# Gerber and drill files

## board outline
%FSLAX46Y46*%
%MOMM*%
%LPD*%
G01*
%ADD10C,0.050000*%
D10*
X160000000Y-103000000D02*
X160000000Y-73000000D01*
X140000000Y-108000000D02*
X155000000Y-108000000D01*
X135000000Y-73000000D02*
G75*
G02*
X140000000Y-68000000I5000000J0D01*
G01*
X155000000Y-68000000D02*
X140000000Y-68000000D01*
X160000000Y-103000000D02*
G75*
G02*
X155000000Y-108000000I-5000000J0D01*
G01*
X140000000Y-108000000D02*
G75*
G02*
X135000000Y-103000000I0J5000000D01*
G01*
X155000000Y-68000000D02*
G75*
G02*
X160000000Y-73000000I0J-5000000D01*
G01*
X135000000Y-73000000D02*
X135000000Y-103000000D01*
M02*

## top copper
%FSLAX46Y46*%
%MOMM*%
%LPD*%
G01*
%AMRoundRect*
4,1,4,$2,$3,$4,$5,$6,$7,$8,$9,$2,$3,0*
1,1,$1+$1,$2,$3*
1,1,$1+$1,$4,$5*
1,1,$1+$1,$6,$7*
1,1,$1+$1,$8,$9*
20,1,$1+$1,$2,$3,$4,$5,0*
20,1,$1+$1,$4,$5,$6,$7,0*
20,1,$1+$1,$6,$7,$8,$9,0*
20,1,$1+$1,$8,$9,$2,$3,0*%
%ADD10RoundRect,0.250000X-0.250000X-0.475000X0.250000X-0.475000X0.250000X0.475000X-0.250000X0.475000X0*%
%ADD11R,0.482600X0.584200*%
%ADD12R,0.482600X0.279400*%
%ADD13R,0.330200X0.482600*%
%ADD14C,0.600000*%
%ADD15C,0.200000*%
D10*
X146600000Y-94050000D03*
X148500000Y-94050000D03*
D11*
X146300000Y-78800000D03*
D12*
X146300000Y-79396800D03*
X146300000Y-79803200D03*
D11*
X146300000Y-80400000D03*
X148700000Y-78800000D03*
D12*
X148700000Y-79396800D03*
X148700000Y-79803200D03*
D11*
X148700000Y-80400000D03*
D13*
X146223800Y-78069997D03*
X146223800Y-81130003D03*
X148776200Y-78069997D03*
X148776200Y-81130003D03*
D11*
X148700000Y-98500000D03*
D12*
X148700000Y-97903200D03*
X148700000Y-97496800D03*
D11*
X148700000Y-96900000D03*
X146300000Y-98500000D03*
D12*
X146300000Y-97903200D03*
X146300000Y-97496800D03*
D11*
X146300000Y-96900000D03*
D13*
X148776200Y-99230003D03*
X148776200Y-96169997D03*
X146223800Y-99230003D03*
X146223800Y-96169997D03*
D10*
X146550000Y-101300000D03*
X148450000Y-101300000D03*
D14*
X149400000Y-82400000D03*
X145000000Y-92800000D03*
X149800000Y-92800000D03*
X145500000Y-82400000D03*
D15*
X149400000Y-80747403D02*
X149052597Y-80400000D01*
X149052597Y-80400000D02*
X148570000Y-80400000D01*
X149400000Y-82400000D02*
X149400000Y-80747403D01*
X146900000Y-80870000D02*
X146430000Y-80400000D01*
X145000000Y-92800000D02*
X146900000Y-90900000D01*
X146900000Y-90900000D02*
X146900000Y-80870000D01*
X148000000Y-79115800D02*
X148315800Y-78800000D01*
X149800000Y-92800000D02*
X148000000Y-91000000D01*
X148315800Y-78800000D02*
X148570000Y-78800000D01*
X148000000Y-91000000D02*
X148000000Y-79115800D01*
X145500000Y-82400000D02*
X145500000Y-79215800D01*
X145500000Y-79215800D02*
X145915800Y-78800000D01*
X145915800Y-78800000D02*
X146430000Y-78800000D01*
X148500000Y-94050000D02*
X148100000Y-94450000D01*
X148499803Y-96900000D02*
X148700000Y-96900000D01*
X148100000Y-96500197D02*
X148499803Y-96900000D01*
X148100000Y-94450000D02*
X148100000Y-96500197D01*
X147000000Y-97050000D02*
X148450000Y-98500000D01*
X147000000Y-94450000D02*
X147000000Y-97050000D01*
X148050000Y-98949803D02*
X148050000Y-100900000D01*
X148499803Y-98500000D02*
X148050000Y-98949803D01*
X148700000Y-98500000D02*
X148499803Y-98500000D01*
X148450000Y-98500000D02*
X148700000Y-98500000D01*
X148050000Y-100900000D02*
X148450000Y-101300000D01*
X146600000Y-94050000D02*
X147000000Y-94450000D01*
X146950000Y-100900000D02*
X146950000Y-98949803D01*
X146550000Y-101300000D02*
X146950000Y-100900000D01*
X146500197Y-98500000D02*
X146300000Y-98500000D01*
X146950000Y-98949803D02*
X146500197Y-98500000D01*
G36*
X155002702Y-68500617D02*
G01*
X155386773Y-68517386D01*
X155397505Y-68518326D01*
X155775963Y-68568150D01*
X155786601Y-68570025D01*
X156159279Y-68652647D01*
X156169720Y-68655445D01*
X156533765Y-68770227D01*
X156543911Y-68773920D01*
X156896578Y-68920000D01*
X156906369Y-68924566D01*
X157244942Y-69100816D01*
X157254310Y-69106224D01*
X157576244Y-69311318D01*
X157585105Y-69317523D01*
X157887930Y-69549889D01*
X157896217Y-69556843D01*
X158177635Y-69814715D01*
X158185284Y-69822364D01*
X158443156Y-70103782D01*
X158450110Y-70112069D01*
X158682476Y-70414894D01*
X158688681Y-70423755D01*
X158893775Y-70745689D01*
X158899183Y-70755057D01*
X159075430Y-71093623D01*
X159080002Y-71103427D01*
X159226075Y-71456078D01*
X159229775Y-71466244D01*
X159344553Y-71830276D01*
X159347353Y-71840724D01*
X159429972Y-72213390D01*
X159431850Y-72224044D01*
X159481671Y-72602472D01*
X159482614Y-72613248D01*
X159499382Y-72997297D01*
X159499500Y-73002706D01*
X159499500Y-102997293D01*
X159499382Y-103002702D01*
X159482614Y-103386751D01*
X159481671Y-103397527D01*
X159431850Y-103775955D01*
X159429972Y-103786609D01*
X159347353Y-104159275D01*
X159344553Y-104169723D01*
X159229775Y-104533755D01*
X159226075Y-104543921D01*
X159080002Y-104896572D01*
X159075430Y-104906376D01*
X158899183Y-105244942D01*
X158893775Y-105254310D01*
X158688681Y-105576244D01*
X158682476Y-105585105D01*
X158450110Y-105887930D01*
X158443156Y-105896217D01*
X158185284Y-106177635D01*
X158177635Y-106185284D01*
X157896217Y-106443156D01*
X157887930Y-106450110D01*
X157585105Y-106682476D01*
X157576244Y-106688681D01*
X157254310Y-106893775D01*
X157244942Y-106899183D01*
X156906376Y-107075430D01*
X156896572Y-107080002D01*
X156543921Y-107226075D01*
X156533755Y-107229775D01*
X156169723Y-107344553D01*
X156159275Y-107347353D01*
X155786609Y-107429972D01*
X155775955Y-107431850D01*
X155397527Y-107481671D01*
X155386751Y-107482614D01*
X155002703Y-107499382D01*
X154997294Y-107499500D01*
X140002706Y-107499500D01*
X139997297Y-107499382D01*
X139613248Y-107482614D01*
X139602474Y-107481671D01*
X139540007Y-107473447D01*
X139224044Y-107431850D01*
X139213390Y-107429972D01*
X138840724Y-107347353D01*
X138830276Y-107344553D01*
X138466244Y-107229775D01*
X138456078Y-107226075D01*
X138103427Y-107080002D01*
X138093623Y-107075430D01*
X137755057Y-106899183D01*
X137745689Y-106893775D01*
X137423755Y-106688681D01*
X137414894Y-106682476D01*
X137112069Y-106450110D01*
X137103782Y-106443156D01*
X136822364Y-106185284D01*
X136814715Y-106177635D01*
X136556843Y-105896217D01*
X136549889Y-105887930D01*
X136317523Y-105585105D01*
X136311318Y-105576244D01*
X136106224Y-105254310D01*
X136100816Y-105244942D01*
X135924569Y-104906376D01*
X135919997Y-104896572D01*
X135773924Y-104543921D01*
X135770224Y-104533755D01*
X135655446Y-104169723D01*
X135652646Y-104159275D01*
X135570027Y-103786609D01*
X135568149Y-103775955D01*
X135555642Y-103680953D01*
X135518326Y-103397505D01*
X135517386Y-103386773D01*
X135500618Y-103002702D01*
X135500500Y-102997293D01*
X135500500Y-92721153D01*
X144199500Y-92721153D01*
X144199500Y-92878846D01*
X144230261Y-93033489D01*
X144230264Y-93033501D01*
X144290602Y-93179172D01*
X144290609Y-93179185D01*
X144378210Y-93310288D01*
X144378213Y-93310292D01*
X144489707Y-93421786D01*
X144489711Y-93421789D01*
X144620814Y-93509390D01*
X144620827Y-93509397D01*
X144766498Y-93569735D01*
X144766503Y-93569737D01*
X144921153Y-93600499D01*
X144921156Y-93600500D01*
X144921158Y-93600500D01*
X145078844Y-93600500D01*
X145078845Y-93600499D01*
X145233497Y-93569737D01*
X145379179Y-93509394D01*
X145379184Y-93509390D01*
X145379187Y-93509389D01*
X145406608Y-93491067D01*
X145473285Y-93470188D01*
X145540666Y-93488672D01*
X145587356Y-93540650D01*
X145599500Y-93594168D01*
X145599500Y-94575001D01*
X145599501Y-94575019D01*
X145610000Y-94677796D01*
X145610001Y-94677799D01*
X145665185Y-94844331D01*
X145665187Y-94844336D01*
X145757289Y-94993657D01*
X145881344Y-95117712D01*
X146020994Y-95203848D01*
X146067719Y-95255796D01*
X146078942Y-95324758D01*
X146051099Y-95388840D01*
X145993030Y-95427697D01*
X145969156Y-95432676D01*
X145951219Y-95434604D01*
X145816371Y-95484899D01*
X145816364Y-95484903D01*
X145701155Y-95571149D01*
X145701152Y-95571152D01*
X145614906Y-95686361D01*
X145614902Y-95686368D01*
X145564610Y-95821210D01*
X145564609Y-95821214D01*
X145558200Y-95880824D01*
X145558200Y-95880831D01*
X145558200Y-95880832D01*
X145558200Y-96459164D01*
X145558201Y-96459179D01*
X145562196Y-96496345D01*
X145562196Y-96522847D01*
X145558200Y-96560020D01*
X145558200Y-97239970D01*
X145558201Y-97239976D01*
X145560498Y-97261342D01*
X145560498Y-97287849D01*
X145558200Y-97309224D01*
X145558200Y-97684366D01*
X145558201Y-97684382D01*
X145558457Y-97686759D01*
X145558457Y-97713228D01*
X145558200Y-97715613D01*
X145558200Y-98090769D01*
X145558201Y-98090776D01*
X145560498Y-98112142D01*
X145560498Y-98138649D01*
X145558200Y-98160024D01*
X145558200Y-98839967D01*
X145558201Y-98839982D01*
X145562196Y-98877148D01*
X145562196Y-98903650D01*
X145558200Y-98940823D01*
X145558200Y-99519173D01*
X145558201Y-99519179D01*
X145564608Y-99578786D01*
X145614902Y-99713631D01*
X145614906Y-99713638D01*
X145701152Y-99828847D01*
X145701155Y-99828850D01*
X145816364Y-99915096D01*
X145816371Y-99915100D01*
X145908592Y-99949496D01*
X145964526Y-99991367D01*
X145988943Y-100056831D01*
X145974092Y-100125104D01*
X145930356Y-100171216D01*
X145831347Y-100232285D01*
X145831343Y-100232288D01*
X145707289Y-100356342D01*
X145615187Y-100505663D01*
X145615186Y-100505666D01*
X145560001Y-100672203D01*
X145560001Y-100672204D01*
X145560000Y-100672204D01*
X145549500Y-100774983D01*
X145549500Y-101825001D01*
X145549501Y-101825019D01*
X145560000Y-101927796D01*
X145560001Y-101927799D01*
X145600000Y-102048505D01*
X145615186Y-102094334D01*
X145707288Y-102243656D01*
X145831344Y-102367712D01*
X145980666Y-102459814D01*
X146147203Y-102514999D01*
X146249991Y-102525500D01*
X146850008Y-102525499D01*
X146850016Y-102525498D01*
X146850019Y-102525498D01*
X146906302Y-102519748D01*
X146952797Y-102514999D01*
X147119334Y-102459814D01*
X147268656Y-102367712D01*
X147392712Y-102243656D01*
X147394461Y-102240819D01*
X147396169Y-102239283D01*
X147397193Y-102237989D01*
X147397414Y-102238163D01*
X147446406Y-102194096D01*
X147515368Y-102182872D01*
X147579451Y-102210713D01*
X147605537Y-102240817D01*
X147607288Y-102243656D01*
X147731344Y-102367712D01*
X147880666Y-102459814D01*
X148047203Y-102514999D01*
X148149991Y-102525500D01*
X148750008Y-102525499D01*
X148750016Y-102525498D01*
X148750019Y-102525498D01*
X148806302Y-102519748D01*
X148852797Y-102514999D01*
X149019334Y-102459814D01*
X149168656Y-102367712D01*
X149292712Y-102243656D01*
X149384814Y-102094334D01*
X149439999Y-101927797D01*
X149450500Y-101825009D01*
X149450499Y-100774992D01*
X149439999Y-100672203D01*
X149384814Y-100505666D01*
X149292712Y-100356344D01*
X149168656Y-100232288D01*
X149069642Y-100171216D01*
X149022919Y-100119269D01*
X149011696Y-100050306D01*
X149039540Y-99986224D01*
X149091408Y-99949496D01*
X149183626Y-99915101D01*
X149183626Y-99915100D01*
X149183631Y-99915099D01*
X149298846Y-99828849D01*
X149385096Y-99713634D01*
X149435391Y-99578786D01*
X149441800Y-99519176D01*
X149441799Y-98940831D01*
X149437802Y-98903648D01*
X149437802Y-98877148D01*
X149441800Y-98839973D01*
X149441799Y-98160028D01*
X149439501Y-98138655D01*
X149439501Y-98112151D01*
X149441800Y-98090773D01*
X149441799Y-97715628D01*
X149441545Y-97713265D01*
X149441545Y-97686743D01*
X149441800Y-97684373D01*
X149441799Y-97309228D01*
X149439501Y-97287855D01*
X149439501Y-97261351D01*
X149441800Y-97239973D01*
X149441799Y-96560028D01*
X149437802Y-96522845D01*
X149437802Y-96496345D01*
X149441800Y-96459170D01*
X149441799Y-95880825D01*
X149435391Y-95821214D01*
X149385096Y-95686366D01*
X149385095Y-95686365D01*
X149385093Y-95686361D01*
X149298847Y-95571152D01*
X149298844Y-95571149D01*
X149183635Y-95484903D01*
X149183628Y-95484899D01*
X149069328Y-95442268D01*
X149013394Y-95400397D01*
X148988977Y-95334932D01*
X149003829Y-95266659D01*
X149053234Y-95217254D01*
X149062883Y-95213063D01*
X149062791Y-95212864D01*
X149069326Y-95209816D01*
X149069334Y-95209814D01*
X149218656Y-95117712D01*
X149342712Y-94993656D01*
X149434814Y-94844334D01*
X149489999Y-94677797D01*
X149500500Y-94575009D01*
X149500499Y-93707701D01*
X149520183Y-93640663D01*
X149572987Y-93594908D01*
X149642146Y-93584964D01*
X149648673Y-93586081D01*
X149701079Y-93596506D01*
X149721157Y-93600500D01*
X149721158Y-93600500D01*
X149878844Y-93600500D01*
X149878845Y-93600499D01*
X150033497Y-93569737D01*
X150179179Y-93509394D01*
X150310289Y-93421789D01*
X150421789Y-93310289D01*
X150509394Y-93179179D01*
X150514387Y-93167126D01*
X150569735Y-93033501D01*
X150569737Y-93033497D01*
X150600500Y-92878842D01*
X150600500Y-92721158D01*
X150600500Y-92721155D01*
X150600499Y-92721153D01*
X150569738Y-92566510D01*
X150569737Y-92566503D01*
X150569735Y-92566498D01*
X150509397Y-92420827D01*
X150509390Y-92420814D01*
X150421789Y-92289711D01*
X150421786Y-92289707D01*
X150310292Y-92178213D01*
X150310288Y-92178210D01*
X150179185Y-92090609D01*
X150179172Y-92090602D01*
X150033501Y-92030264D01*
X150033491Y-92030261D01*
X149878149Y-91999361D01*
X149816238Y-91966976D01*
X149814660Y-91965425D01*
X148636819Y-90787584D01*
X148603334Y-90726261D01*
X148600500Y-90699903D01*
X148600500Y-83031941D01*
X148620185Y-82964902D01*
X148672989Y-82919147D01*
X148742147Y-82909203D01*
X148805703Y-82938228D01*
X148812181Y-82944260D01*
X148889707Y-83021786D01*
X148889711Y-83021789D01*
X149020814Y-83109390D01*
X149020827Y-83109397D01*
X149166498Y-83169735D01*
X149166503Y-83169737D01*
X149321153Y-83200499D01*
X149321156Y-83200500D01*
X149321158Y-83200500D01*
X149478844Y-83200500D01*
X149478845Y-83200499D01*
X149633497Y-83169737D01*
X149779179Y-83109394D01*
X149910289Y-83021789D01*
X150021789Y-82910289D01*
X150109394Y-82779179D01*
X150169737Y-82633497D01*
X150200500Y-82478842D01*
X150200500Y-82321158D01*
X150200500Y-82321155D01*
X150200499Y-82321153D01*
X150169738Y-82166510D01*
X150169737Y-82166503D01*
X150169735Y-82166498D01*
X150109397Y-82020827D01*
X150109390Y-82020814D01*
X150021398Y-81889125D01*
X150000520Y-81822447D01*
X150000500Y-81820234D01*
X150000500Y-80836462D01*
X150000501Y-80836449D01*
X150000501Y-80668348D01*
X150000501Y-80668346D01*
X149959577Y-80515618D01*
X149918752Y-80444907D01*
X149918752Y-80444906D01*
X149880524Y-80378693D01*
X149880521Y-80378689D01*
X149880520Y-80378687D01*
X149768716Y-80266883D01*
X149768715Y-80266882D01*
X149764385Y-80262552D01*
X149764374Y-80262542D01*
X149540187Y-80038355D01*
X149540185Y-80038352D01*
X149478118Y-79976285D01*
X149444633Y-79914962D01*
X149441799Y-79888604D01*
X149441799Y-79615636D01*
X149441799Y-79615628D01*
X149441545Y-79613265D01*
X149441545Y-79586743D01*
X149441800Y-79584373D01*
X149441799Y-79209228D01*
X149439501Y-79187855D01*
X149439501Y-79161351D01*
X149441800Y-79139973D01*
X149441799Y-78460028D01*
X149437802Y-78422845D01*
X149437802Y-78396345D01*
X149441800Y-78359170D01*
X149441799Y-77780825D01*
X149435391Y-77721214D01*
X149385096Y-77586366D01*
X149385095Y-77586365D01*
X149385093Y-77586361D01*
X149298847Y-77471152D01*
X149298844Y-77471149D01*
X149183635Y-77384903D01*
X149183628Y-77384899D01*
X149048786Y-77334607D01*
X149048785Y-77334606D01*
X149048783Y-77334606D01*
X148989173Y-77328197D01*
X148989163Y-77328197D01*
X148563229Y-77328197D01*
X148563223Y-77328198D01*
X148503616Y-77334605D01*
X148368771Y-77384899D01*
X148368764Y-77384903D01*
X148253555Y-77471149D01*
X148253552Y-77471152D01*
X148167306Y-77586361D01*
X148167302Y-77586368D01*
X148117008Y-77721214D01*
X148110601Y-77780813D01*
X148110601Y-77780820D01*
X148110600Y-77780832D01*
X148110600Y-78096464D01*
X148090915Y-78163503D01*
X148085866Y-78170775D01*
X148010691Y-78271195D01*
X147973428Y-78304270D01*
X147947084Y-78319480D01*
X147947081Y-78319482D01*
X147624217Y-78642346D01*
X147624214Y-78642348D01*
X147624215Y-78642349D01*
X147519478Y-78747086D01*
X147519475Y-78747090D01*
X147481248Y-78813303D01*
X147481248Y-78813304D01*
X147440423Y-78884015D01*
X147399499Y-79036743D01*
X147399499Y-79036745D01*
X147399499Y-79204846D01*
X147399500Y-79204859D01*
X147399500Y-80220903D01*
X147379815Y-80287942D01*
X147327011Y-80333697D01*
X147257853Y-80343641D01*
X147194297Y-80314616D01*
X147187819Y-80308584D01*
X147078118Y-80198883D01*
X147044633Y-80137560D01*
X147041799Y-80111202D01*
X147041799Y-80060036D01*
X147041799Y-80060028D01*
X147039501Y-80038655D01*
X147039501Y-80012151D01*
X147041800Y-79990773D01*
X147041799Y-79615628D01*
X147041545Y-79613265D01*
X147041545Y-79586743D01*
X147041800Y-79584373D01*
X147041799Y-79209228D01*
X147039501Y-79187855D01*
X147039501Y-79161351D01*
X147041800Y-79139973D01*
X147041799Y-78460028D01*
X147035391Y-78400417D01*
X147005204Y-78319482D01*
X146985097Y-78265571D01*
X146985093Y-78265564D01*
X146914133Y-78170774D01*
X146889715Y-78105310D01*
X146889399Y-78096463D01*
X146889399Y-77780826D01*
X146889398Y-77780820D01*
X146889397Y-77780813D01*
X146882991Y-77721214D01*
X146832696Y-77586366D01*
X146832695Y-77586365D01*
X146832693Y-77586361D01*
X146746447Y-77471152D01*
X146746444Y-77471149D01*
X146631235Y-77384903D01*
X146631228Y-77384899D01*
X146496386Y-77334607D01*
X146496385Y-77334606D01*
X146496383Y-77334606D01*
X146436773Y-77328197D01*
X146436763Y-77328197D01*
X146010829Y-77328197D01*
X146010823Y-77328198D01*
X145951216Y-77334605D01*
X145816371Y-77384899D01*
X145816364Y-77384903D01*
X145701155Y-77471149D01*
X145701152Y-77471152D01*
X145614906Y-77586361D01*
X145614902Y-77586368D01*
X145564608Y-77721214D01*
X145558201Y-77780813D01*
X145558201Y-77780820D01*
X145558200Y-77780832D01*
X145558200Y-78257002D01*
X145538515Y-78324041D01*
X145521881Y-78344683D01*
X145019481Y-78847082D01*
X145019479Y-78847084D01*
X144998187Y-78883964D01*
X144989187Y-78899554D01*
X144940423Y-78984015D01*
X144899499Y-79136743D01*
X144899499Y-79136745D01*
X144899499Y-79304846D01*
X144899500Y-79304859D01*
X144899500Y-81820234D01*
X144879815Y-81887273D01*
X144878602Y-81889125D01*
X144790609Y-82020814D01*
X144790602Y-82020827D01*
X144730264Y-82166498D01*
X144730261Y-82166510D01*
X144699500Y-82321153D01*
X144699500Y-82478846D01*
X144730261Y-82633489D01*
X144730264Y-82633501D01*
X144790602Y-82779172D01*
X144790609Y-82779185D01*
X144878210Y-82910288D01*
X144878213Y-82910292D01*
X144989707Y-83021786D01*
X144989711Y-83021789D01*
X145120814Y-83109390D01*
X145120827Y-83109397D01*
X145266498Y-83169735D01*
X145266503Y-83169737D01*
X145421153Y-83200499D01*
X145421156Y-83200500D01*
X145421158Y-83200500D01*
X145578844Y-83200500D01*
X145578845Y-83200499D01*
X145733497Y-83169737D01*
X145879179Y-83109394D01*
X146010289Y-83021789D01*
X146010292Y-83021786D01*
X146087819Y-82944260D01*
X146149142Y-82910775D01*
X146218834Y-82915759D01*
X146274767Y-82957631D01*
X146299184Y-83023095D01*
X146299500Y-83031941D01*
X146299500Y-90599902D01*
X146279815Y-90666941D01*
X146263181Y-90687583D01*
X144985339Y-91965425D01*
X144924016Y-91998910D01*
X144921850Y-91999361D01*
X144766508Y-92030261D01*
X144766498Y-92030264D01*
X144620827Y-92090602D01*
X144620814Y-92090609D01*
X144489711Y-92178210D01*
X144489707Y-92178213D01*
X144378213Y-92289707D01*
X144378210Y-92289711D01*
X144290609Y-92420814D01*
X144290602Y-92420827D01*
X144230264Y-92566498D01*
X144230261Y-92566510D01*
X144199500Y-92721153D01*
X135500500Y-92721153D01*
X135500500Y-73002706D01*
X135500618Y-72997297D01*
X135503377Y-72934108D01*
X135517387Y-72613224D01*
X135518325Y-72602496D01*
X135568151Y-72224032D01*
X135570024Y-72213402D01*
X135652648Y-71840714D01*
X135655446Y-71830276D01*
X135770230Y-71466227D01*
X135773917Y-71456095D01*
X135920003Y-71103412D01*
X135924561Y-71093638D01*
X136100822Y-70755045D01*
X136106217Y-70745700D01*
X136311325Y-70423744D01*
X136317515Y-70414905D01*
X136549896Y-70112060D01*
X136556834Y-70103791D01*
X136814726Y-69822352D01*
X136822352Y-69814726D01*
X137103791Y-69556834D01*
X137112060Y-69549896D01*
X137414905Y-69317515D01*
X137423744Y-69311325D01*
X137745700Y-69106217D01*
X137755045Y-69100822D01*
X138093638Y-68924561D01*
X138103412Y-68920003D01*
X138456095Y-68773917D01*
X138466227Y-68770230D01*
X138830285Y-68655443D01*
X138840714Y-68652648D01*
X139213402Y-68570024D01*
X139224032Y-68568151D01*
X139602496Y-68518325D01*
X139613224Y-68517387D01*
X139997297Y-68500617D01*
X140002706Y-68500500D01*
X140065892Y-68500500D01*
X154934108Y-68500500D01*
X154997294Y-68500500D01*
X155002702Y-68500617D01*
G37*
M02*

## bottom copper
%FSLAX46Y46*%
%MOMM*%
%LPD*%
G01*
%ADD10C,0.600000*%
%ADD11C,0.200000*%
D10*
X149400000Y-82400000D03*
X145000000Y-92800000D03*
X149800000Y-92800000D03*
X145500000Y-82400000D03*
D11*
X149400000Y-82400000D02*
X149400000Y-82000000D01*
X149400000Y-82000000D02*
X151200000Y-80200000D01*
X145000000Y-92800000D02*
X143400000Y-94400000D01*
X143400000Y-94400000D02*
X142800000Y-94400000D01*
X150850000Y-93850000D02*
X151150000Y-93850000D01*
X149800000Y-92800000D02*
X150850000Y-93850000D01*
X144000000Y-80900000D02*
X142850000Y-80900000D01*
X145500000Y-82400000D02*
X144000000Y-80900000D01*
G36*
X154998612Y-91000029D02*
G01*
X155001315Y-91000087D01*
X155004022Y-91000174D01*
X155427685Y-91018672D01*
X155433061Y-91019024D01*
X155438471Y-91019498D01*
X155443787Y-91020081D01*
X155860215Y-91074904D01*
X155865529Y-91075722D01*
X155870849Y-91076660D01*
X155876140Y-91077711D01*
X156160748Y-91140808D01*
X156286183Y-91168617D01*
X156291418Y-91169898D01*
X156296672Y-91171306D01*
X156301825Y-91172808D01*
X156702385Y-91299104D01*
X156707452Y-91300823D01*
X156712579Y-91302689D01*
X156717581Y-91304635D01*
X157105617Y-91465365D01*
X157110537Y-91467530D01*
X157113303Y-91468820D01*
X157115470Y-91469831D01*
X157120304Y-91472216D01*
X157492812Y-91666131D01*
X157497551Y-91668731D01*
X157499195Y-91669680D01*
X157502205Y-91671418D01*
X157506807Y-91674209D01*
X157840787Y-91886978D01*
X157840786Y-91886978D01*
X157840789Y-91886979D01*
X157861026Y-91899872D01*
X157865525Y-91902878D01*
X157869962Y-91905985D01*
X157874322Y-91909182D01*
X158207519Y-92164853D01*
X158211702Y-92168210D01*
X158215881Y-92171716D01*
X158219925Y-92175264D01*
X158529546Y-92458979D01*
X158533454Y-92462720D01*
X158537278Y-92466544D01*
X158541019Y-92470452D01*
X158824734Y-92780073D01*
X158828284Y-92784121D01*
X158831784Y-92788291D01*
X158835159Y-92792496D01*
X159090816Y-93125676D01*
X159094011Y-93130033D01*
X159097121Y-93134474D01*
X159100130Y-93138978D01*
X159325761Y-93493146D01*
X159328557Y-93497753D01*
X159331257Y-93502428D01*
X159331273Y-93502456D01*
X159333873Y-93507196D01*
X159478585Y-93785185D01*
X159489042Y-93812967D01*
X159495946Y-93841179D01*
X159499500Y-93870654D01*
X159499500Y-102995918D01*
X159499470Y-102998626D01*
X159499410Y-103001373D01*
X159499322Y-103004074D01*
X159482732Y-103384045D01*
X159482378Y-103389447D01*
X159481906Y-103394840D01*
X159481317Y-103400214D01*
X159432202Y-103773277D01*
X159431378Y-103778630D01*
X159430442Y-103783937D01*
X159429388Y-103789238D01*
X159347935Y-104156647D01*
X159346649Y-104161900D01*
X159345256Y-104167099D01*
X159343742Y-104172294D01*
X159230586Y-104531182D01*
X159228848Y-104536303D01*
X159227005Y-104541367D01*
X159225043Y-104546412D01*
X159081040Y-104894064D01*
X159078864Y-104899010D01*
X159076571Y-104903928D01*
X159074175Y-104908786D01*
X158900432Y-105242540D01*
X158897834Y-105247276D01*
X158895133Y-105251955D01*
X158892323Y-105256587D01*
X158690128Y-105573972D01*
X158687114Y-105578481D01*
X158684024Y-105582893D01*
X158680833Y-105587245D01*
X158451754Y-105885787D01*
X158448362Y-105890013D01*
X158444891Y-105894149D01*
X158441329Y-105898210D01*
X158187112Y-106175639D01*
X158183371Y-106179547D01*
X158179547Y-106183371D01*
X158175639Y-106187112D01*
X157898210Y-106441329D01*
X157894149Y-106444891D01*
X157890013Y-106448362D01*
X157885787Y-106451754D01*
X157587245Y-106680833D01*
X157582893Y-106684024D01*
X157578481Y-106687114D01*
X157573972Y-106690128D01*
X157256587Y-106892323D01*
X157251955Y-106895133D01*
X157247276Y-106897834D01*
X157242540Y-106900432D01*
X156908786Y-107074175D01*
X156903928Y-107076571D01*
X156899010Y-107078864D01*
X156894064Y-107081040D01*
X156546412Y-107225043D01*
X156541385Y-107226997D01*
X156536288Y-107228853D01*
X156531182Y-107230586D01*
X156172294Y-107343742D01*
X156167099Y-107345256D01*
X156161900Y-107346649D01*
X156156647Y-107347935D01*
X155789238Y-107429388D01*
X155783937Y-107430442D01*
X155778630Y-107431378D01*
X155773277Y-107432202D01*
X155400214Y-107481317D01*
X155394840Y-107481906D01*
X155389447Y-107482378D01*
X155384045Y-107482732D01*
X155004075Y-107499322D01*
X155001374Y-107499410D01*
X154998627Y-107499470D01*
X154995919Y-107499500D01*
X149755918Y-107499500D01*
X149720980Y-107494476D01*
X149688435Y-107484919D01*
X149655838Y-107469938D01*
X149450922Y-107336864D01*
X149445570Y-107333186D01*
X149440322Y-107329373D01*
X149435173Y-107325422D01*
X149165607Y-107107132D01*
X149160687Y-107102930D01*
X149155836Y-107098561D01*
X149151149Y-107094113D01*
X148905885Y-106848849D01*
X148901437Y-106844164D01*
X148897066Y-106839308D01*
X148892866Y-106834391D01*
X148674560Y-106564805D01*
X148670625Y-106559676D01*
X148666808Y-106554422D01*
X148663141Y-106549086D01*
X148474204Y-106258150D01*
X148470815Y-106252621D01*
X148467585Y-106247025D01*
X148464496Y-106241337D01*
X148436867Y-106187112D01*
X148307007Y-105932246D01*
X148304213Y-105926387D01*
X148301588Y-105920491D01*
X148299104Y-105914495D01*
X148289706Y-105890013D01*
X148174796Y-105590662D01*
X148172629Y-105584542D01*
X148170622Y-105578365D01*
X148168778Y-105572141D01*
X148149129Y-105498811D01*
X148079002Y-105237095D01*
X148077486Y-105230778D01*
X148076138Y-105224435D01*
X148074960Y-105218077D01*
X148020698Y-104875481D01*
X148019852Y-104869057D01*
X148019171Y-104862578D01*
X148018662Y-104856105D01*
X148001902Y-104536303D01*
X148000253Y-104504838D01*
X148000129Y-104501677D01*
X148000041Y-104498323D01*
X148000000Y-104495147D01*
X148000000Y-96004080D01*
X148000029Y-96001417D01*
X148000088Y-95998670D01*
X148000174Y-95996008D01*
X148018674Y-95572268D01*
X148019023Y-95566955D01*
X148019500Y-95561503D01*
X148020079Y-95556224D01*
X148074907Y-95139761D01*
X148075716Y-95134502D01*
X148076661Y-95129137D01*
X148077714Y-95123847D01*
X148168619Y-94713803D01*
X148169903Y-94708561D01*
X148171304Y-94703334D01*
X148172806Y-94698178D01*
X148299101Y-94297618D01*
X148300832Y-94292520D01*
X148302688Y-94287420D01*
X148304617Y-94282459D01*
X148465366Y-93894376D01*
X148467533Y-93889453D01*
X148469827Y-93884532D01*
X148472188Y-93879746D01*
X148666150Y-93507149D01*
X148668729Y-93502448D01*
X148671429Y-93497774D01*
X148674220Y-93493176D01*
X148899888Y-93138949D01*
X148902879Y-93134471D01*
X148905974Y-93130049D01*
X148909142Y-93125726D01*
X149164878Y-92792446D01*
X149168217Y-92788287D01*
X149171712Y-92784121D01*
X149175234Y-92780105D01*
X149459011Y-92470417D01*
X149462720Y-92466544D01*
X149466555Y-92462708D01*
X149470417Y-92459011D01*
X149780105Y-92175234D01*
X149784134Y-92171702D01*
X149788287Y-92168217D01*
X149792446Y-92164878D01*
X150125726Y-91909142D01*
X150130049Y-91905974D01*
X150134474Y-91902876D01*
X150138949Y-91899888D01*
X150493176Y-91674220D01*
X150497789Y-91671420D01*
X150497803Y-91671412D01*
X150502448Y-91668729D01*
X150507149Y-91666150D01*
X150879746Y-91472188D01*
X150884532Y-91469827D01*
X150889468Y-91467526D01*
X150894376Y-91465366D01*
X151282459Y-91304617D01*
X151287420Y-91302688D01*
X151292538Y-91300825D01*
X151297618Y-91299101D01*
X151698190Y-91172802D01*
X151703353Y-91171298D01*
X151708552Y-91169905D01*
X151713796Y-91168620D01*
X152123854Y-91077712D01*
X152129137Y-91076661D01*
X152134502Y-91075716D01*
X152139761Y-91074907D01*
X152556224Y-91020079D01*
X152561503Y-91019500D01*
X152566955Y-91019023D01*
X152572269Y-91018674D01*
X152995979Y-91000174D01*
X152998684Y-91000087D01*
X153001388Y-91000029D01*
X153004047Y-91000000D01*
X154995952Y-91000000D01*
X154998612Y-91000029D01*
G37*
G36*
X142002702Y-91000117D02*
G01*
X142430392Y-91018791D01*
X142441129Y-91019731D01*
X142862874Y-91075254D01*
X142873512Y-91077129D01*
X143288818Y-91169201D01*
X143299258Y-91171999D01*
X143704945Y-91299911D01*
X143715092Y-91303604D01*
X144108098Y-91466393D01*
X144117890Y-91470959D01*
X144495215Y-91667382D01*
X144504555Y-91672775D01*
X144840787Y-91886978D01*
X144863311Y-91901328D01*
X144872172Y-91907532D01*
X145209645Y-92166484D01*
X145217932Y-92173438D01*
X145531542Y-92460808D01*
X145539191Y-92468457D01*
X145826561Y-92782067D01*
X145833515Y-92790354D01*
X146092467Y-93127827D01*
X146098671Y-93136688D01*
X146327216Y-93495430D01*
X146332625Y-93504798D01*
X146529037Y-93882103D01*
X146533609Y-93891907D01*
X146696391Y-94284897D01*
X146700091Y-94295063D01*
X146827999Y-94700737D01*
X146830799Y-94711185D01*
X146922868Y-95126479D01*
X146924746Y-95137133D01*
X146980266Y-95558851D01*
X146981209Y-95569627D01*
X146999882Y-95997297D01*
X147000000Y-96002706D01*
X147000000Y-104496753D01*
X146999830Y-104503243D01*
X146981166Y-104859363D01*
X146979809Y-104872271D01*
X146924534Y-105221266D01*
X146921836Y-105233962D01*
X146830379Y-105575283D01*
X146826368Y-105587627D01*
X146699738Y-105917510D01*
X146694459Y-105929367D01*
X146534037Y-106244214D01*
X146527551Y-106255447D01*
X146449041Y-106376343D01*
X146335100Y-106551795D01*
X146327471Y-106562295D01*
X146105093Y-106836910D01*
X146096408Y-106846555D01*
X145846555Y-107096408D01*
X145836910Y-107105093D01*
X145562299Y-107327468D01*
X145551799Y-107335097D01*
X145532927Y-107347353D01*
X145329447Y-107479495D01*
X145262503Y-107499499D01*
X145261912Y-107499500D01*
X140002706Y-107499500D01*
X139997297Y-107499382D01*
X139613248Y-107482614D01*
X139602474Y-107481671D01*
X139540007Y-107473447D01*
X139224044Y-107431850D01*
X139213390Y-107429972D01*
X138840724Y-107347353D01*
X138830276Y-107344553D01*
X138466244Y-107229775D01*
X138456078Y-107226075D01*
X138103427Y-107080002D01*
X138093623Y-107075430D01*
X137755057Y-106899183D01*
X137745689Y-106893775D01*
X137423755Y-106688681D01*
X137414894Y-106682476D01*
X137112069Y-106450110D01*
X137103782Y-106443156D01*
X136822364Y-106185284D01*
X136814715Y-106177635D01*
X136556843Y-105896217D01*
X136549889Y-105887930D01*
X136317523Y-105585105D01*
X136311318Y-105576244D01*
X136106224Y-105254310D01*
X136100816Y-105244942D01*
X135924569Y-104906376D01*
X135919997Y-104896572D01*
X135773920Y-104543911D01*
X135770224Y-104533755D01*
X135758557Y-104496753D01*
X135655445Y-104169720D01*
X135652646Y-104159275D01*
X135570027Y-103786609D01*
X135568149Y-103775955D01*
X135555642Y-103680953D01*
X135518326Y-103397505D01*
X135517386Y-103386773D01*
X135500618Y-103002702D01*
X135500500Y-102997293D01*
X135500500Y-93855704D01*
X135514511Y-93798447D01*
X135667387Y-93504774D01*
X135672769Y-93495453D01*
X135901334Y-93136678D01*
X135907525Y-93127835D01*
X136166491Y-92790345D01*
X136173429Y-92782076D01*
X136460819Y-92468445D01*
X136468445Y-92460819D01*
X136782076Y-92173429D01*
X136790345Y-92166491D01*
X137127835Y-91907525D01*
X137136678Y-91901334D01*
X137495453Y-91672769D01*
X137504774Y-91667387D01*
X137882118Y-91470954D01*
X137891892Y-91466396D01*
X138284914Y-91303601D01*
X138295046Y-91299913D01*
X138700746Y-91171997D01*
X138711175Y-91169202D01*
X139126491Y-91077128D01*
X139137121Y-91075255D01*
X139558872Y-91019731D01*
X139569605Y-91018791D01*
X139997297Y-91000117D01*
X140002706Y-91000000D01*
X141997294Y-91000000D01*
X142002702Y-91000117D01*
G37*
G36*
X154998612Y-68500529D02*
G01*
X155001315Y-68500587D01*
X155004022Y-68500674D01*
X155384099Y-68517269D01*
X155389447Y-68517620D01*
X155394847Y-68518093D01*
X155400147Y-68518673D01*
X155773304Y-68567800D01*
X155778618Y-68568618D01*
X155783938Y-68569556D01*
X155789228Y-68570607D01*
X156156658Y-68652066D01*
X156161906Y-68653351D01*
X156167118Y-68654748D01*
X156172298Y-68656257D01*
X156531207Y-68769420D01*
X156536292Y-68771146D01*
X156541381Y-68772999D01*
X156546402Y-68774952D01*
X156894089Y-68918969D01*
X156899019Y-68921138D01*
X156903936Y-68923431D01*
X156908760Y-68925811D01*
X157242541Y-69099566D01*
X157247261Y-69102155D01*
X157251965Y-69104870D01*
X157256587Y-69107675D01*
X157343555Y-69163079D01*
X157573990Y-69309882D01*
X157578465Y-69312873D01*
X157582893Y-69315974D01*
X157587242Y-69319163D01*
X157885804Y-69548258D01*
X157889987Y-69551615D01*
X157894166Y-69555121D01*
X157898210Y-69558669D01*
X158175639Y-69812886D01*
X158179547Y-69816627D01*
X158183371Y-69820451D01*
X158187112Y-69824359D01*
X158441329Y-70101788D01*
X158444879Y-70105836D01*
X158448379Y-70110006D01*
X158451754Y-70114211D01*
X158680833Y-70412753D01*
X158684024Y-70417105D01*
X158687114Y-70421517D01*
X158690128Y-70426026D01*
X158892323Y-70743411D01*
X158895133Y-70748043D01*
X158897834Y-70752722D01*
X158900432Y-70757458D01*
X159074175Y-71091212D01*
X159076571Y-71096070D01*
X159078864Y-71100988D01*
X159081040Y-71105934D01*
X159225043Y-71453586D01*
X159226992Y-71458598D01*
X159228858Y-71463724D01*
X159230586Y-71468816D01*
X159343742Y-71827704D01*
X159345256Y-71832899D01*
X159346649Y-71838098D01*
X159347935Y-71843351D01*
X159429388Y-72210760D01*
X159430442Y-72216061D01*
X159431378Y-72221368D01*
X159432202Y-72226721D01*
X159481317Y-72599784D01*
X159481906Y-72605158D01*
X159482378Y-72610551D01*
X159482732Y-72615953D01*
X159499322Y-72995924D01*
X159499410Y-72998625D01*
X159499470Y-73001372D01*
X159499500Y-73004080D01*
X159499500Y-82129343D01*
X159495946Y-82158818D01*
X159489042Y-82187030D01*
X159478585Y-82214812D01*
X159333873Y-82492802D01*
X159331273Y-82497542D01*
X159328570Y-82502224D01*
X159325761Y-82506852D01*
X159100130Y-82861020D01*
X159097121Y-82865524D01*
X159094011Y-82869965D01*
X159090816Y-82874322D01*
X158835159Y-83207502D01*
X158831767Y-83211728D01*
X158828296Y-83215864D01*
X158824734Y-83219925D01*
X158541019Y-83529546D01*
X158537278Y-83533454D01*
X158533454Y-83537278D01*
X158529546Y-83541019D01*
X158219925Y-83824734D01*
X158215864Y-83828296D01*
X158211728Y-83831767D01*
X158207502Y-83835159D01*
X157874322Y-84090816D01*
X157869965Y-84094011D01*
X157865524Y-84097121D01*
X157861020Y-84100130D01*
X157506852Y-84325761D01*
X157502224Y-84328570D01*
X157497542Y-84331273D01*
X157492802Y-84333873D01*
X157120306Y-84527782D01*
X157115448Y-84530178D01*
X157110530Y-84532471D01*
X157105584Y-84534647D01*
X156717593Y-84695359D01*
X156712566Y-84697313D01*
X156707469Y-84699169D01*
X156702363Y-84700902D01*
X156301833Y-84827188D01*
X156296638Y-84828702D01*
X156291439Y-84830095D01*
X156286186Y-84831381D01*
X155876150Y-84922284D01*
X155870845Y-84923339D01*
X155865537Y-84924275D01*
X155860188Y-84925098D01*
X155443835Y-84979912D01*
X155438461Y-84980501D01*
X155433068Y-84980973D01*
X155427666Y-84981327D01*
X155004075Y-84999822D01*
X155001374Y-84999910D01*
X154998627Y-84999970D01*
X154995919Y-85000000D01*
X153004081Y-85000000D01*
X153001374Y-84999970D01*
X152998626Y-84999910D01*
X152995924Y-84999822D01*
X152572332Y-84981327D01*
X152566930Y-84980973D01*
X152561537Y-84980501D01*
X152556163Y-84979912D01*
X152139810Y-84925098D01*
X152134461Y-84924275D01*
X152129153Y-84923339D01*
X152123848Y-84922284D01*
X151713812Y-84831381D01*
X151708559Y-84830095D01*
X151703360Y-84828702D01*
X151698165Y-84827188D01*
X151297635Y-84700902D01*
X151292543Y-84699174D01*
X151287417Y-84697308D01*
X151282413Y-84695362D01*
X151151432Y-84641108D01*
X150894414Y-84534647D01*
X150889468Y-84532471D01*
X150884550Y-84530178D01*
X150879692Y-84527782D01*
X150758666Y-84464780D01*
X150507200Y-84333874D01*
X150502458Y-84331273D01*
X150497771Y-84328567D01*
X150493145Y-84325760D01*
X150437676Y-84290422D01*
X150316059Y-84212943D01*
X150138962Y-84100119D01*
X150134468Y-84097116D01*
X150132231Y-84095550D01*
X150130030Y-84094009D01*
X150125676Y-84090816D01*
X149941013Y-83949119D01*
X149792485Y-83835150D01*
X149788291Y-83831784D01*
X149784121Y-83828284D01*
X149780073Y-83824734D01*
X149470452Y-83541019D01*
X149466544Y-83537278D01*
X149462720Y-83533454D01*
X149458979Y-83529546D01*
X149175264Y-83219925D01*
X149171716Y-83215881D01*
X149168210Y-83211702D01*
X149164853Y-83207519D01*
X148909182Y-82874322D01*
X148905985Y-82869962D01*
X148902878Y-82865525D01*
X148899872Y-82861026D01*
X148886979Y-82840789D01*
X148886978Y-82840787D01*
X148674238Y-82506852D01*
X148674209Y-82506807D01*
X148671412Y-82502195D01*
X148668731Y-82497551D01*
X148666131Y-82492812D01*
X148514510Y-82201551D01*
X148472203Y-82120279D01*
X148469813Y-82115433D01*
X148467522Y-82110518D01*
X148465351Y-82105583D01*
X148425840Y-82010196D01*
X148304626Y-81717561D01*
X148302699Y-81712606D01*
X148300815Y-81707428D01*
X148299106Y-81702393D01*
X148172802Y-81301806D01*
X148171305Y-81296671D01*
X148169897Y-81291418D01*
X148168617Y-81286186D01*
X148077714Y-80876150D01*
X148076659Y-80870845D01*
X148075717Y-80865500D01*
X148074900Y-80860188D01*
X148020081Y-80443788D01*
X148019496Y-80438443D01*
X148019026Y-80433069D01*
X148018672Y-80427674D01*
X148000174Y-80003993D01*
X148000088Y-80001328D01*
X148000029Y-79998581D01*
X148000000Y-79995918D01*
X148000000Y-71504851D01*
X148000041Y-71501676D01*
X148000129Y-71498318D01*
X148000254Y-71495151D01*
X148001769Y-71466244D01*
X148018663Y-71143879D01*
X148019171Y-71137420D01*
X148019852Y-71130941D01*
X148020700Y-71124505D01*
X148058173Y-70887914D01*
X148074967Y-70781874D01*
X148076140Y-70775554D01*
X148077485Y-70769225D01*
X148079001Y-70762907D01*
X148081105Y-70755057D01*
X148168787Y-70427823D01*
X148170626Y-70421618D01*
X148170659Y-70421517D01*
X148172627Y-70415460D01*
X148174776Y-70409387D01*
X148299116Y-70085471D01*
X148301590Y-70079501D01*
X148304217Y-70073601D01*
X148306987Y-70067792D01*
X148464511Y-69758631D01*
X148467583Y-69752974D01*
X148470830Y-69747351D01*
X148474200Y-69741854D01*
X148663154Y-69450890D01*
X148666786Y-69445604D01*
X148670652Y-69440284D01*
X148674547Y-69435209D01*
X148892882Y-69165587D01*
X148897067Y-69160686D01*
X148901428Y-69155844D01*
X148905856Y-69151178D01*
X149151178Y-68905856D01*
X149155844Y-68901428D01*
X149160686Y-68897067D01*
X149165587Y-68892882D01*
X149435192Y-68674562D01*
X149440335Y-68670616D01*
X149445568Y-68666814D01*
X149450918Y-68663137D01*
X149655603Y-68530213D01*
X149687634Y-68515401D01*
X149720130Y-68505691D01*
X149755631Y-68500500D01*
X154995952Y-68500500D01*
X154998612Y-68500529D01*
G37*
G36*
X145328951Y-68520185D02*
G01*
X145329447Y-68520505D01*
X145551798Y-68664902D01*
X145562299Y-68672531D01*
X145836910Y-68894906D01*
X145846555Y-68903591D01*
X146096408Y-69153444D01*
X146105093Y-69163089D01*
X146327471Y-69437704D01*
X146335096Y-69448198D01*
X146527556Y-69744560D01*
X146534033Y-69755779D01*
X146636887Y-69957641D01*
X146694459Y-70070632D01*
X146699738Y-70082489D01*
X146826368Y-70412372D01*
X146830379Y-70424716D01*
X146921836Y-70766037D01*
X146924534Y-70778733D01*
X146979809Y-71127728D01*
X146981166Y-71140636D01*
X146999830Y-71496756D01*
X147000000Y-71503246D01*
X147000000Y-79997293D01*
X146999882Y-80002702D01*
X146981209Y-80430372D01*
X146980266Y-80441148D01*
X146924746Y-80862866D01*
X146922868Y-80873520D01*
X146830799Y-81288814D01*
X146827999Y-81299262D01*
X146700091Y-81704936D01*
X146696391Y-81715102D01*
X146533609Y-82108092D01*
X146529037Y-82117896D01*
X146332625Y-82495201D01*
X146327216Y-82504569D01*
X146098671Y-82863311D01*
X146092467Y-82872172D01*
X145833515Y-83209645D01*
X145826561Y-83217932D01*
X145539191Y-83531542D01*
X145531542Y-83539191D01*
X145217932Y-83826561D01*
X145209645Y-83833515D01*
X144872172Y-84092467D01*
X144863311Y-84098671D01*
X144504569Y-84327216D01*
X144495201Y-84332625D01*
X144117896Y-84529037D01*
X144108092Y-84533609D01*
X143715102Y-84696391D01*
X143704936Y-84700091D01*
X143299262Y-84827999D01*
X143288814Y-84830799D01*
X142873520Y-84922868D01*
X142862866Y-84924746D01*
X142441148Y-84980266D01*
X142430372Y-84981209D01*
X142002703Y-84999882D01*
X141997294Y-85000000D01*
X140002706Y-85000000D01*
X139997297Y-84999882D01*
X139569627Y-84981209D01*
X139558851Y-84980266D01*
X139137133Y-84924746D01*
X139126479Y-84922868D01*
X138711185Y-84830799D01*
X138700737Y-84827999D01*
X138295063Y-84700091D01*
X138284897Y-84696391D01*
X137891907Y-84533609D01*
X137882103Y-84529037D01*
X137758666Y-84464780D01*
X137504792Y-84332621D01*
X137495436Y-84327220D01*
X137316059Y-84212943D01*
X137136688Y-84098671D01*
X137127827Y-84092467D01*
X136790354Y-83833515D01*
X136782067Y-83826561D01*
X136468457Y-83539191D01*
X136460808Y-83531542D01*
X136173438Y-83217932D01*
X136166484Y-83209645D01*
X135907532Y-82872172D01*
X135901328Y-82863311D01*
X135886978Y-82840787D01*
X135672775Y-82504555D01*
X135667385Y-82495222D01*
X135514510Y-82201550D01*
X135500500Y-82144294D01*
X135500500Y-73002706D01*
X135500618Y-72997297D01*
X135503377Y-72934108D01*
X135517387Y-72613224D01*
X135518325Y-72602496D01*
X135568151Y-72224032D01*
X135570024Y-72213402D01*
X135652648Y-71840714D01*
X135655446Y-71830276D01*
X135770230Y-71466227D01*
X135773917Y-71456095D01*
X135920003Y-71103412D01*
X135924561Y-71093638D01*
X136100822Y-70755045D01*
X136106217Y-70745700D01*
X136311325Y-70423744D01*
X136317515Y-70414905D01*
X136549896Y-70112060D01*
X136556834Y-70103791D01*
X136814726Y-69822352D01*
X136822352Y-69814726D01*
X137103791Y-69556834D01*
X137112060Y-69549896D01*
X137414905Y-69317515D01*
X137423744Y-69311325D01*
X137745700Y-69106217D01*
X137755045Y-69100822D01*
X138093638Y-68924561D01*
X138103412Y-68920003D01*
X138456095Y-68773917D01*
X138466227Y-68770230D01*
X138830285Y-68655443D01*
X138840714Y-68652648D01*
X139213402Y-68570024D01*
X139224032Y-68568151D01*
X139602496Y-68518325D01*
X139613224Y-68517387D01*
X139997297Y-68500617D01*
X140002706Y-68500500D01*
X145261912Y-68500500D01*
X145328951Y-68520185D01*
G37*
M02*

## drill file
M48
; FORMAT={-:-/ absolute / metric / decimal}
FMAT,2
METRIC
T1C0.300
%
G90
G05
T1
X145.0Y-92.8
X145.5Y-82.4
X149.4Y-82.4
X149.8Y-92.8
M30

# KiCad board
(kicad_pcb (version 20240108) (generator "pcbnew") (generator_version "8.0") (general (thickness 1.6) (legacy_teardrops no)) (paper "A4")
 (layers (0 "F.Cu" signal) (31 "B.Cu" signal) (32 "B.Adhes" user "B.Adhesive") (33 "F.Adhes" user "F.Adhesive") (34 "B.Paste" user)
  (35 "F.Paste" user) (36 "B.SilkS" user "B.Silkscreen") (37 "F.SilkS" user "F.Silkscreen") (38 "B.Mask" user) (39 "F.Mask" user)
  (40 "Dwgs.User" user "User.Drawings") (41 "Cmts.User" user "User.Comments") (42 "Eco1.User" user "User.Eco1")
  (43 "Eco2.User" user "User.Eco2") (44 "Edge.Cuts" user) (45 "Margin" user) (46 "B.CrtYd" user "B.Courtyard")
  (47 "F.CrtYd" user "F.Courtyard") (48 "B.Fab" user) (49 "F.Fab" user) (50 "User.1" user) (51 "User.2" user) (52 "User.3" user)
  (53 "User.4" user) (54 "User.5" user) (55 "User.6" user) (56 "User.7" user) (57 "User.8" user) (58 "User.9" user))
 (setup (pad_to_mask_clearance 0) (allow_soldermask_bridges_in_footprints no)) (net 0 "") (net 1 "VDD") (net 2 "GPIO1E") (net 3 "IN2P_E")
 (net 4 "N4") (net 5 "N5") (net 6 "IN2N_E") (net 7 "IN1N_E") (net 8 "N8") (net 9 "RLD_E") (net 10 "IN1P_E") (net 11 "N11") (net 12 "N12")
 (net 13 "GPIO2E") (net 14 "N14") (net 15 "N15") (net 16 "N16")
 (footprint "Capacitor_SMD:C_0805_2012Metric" (layer "F.Cu") (at 147.55 94.05)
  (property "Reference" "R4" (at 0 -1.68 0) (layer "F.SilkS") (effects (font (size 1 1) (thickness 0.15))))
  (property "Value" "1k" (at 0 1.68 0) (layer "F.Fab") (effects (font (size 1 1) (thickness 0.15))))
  (pad "1" smd roundrect (at -0.95 0) (size 1 1.45) (layers "F.Cu" "F.Paste" "F.Mask") (roundrect_rratio 0.25) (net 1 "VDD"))
  (pad "2" smd roundrect (at 0.95 0) (size 1 1.45) (layers "F.Cu" "F.Paste" "F.Mask") (roundrect_rratio 0.25) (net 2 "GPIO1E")))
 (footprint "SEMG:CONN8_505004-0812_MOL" (layer "F.Cu") (at 147.5 79.6 90)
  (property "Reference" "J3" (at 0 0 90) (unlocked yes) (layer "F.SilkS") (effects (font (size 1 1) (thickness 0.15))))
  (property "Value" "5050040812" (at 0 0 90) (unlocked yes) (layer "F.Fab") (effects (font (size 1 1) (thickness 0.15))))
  (pad "1" smd rect (at 0.8 -1.2 90) (size 0.5842 0.4826) (layers "F.Cu" "F.Paste" "F.Mask") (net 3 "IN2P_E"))
  (pad "2" smd rect (at 0.2032 -1.2 90) (size 0.2794 0.4826) (layers "F.Cu" "F.Paste" "F.Mask") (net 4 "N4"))
  (pad "3" smd rect (at -0.2032 -1.2 90) (size 0.2794 0.4826) (layers "F.Cu" "F.Paste" "F.Mask") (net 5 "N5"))
  (pad "4" smd rect (at -0.8 -1.2 90) (size 0.5842 0.4826) (layers "F.Cu" "F.Paste" "F.Mask") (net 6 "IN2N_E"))
  (pad "5" smd rect (at 0.8 1.2 90) (size 0.5842 0.4826) (layers "F.Cu" "F.Paste" "F.Mask") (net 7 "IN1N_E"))
  (pad "6" smd rect (at 0.2032 1.2 90) (size 0.2794 0.4826) (layers "F.Cu" "F.Paste" "F.Mask") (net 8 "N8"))
  (pad "7" smd rect (at -0.2032 1.2 90) (size 0.2794 0.4826) (layers "F.Cu" "F.Paste" "F.Mask") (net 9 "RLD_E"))
  (pad "8" smd rect (at -0.8 1.2 90) (size 0.5842 0.4826) (layers "F.Cu" "F.Paste" "F.Mask") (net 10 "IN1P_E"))
  (pad "9" smd rect (at 1.530003 -1.2762 90) (size 0.4826 0.3302) (layers "F.Cu" "F.Paste" "F.Mask"))
  (pad "10" smd rect (at -1.530003 -1.2762 90) (size 0.4826 0.3302) (layers "F.Cu" "F.Paste" "F.Mask"))
  (pad "11" smd rect (at 1.530003 1.2762 90) (size 0.4826 0.3302) (layers "F.Cu" "F.Paste" "F.Mask"))
  (pad "12" smd rect (at -1.530003 1.2762 90) (size 0.4826 0.3302) (layers "F.Cu" "F.Paste" "F.Mask")))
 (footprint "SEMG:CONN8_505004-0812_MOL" (layer "F.Cu") (at 147.5 97.7 -90)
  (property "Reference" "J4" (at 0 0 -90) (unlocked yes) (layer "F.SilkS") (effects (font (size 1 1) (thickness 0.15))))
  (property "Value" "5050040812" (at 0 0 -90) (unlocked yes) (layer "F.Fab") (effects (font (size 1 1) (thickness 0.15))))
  (pad "1" smd rect (at 0.8 -1.2 270) (size 0.5842 0.4826) (layers "F.Cu" "F.Paste" "F.Mask") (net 1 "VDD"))
  (pad "2" smd rect (at 0.2032 -1.2 270) (size 0.2794 0.4826) (layers "F.Cu" "F.Paste" "F.Mask") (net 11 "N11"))
  (pad "3" smd rect (at -0.2032 -1.2 270) (size 0.2794 0.4826) (layers "F.Cu" "F.Paste" "F.Mask") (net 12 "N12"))
  (pad "4" smd rect (at -0.8 -1.2 270) (size 0.5842 0.4826) (layers "F.Cu" "F.Paste" "F.Mask") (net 2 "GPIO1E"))
  (pad "5" smd rect (at 0.8 1.2 270) (size 0.5842 0.4826) (layers "F.Cu" "F.Paste" "F.Mask") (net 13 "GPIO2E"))
  (pad "6" smd rect (at 0.2032 1.2 270) (size 0.2794 0.4826) (layers "F.Cu" "F.Paste" "F.Mask") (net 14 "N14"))
  (pad "7" smd rect (at -0.2032 1.2 270) (size 0.2794 0.4826) (layers "F.Cu" "F.Paste" "F.Mask") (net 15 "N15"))
  (pad "8" smd rect (at -0.8 1.2 270) (size 0.5842 0.4826) (layers "F.Cu" "F.Paste" "F.Mask") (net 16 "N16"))
  (pad "9" smd rect (at 1.530003 -1.2762 270) (size 0.4826 0.3302) (layers "F.Cu" "F.Paste" "F.Mask"))
  (pad "10" smd rect (at -1.530003 -1.2762 270) (size 0.4826 0.3302) (layers "F.Cu" "F.Paste" "F.Mask"))
  (pad "11" smd rect (at 1.530003 1.2762 270) (size 0.4826 0.3302) (layers "F.Cu" "F.Paste" "F.Mask"))
  (pad "12" smd rect (at -1.530003 1.2762 270) (size 0.4826 0.3302) (layers "F.Cu" "F.Paste" "F.Mask")))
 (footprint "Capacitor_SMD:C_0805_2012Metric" (layer "F.Cu") (at 147.5 101.3)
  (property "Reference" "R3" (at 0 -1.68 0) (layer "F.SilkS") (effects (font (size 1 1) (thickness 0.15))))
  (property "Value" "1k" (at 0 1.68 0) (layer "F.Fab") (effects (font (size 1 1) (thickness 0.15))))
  (pad "1" smd roundrect (at -0.95 0) (size 1 1.45) (layers "F.Cu" "F.Paste" "F.Mask") (roundrect_rratio 0.25) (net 13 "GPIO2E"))
  (pad "2" smd roundrect (at 0.95 0) (size 1 1.45) (layers "F.Cu" "F.Paste" "F.Mask") (roundrect_rratio 0.25) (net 1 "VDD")))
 (gr_line (start 160 103) (end 160 73) (stroke (width 0.05) (type default)) (layer "Edge.Cuts"))
 (gr_line (start 140 108) (end 155 108) (stroke (width 0.05) (type default)) (layer "Edge.Cuts"))
 (gr_arc (start 135 73) (mid 136.464466 69.464466) (end 140 68) (stroke (width 0.05) (type default)) (layer "Edge.Cuts"))
 (gr_line (start 155 68) (end 140 68) (stroke (width 0.05) (type default)) (layer "Edge.Cuts"))
 (gr_arc (start 160 103) (mid 158.535534 106.535534) (end 155 108) (stroke (width 0.05) (type default)) (layer "Edge.Cuts"))
 (gr_arc (start 140 108) (mid 136.464466 106.535534) (end 135 103) (stroke (width 0.05) (type default)) (layer "Edge.Cuts"))
 (gr_arc (start 155 68) (mid 158.535534 69.464466) (end 160 73) (stroke (width 0.05) (type default)) (layer "Edge.Cuts"))
 (gr_line (start 135 73) (end 135 103) (stroke (width 0.05) (type default)) (layer "Edge.Cuts"))
 (segment (start 149.4 80.747403) (end 149.052597 80.4) (width 0.2) (layer "F.Cu") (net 10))
 (segment (start 149.052597 80.4) (end 148.57 80.4) (width 0.2) (layer "F.Cu") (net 10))
 (segment (start 149.4 82.4) (end 149.4 80.747403) (width 0.2) (layer "F.Cu") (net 10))
 (via (at 149.4 82.4) (size 0.6) (drill 0.3) (layers "F.Cu" "B.Cu") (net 10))
 (segment (start 149.4 82.4) (end 149.4 82) (width 0.2) (layer "B.Cu") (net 10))
 (segment (start 149.4 82) (end 151.2 80.2) (width 0.2) (layer "B.Cu") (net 10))
 (segment (start 146.9 80.87) (end 146.43 80.4) (width 0.2) (layer "F.Cu") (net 6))
 (segment (start 145 92.8) (end 146.9 90.9) (width 0.2) (layer "F.Cu") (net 6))
 (segment (start 146.9 90.9) (end 146.9 80.87) (width 0.2) (layer "F.Cu") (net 6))
 (via (at 145 92.8) (size 0.6) (drill 0.3) (layers "F.Cu" "B.Cu") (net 6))
 (segment (start 145 92.8) (end 143.4 94.4) (width 0.2) (layer "B.Cu") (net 6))
 (segment (start 143.4 94.4) (end 142.8 94.4) (width 0.2) (layer "B.Cu") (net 6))
 (segment (start 148 79.1158) (end 148.3158 78.8) (width 0.2) (layer "F.Cu") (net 7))
 (segment (start 149.8 92.8) (end 148 91) (width 0.2) (layer "F.Cu") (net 7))
 (segment (start 148.3158 78.8) (end 148.57 78.8) (width 0.2) (layer "F.Cu") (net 7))
 (segment (start 148 91) (end 148 79.1158) (width 0.2) (layer "F.Cu") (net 7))
 (via (at 149.8 92.8) (size 0.6) (drill 0.3) (layers "F.Cu" "B.Cu") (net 7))
 (segment (start 150.85 93.85) (end 151.15 93.85) (width 0.2) (layer "B.Cu") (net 7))
 (segment (start 149.8 92.8) (end 150.85 93.85) (width 0.2) (layer "B.Cu") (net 7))
 (segment (start 145.5 82.4) (end 145.5 79.2158) (width 0.2) (layer "F.Cu") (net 3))
 (segment (start 145.5 79.2158) (end 145.9158 78.8) (width 0.2) (layer "F.Cu") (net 3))
 (segment (start 145.9158 78.8) (end 146.43 78.8) (width 0.2) (layer "F.Cu") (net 3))
 (via (at 145.5 82.4) (size 0.6) (drill 0.3) (layers "F.Cu" "B.Cu") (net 3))
 (segment (start 144 80.9) (end 142.85 80.9) (width 0.2) (layer "B.Cu") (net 3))
 (segment (start 145.5 82.4) (end 144 80.9) (width 0.2) (layer "B.Cu") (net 3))
 (segment (start 148.5 94.05) (end 148.1 94.45) (width 0.2) (layer "F.Cu") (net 2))
 (segment (start 148.499803 96.9) (end 148.7 96.9) (width 0.2) (layer "F.Cu") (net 2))
 (segment (start 148.1 96.500197) (end 148.499803 96.9) (width 0.2) (layer "F.Cu") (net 2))
 (segment (start 148.1 94.45) (end 148.1 96.500197) (width 0.2) (layer "F.Cu") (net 2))
 (segment (start 147 97.05) (end 148.45 98.5) (width 0.2) (layer "F.Cu") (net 1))
 (segment (start 147 94.45) (end 147 97.05) (width 0.2) (layer "F.Cu") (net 1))
 (segment (start 148.05 98.949803) (end 148.05 100.9) (width 0.2) (layer "F.Cu") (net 1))
 (segment (start 148.499803 98.5) (end 148.05 98.949803) (width 0.2) (layer "F.Cu") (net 1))
 (segment (start 148.7 98.5) (end 148.499803 98.5) (width 0.2) (layer "F.Cu") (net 1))
 (segment (start 148.45 98.5) (end 148.7 98.5) (width 0.2) (layer "F.Cu") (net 1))
 (segment (start 148.05 100.9) (end 148.45 101.3) (width 0.2) (layer "F.Cu") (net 1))
 (segment (start 146.6 94.05) (end 147 94.45) (width 0.2) (layer "F.Cu") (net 1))
 (segment (start 146.95 100.9) (end 146.95 98.949803) (width 0.2) (layer "F.Cu") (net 13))
 (segment (start 146.55 101.3) (end 146.95 100.9) (width 0.2) (layer "F.Cu") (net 13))
 (segment (start 146.500197 98.5) (end 146.3 98.5) (width 0.2) (layer "F.Cu") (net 13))
 (segment (start 146.95 98.949803) (end 146.500197 98.5) (width 0.2) (layer "F.Cu") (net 13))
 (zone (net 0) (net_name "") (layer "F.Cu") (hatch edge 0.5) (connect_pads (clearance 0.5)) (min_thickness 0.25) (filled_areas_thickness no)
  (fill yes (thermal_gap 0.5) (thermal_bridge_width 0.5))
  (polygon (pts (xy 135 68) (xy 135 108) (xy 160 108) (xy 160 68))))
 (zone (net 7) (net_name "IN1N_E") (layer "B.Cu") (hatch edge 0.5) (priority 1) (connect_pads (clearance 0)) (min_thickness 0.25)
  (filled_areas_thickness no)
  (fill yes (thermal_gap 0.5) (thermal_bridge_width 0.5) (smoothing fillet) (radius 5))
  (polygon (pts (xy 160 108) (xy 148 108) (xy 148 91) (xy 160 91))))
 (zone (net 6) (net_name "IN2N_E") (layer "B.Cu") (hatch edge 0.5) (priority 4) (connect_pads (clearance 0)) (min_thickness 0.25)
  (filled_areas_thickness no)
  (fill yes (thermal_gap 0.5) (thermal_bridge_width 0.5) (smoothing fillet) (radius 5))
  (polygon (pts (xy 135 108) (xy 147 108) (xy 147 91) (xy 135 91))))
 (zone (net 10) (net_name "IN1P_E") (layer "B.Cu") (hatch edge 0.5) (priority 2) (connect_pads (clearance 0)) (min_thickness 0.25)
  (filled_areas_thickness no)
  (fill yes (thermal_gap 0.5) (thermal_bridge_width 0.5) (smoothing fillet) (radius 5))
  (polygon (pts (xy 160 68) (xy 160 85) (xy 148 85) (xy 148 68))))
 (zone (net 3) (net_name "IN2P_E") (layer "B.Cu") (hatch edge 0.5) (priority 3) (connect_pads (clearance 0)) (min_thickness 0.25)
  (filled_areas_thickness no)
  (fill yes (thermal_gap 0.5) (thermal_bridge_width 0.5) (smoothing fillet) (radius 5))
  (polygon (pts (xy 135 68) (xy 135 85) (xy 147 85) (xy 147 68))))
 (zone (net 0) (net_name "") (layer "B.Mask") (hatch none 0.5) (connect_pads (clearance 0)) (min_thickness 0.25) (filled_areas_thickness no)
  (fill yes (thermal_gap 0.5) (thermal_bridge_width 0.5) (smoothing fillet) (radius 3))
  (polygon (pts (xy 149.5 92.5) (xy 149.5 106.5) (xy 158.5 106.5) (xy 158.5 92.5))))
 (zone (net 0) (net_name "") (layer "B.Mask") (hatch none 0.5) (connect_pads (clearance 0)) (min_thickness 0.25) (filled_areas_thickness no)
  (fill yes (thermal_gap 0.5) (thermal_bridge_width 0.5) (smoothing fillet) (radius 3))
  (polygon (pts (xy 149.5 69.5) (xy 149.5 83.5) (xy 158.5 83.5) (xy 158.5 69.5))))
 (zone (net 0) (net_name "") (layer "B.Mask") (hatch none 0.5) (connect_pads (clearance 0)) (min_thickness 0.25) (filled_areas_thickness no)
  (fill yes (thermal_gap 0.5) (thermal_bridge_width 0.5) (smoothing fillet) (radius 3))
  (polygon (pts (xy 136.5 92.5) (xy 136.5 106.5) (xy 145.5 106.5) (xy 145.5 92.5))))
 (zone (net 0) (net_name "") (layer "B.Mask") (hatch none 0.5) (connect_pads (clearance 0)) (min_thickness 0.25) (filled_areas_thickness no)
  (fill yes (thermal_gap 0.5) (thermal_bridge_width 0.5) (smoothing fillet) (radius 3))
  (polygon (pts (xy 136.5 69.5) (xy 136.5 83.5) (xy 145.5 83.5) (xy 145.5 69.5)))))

